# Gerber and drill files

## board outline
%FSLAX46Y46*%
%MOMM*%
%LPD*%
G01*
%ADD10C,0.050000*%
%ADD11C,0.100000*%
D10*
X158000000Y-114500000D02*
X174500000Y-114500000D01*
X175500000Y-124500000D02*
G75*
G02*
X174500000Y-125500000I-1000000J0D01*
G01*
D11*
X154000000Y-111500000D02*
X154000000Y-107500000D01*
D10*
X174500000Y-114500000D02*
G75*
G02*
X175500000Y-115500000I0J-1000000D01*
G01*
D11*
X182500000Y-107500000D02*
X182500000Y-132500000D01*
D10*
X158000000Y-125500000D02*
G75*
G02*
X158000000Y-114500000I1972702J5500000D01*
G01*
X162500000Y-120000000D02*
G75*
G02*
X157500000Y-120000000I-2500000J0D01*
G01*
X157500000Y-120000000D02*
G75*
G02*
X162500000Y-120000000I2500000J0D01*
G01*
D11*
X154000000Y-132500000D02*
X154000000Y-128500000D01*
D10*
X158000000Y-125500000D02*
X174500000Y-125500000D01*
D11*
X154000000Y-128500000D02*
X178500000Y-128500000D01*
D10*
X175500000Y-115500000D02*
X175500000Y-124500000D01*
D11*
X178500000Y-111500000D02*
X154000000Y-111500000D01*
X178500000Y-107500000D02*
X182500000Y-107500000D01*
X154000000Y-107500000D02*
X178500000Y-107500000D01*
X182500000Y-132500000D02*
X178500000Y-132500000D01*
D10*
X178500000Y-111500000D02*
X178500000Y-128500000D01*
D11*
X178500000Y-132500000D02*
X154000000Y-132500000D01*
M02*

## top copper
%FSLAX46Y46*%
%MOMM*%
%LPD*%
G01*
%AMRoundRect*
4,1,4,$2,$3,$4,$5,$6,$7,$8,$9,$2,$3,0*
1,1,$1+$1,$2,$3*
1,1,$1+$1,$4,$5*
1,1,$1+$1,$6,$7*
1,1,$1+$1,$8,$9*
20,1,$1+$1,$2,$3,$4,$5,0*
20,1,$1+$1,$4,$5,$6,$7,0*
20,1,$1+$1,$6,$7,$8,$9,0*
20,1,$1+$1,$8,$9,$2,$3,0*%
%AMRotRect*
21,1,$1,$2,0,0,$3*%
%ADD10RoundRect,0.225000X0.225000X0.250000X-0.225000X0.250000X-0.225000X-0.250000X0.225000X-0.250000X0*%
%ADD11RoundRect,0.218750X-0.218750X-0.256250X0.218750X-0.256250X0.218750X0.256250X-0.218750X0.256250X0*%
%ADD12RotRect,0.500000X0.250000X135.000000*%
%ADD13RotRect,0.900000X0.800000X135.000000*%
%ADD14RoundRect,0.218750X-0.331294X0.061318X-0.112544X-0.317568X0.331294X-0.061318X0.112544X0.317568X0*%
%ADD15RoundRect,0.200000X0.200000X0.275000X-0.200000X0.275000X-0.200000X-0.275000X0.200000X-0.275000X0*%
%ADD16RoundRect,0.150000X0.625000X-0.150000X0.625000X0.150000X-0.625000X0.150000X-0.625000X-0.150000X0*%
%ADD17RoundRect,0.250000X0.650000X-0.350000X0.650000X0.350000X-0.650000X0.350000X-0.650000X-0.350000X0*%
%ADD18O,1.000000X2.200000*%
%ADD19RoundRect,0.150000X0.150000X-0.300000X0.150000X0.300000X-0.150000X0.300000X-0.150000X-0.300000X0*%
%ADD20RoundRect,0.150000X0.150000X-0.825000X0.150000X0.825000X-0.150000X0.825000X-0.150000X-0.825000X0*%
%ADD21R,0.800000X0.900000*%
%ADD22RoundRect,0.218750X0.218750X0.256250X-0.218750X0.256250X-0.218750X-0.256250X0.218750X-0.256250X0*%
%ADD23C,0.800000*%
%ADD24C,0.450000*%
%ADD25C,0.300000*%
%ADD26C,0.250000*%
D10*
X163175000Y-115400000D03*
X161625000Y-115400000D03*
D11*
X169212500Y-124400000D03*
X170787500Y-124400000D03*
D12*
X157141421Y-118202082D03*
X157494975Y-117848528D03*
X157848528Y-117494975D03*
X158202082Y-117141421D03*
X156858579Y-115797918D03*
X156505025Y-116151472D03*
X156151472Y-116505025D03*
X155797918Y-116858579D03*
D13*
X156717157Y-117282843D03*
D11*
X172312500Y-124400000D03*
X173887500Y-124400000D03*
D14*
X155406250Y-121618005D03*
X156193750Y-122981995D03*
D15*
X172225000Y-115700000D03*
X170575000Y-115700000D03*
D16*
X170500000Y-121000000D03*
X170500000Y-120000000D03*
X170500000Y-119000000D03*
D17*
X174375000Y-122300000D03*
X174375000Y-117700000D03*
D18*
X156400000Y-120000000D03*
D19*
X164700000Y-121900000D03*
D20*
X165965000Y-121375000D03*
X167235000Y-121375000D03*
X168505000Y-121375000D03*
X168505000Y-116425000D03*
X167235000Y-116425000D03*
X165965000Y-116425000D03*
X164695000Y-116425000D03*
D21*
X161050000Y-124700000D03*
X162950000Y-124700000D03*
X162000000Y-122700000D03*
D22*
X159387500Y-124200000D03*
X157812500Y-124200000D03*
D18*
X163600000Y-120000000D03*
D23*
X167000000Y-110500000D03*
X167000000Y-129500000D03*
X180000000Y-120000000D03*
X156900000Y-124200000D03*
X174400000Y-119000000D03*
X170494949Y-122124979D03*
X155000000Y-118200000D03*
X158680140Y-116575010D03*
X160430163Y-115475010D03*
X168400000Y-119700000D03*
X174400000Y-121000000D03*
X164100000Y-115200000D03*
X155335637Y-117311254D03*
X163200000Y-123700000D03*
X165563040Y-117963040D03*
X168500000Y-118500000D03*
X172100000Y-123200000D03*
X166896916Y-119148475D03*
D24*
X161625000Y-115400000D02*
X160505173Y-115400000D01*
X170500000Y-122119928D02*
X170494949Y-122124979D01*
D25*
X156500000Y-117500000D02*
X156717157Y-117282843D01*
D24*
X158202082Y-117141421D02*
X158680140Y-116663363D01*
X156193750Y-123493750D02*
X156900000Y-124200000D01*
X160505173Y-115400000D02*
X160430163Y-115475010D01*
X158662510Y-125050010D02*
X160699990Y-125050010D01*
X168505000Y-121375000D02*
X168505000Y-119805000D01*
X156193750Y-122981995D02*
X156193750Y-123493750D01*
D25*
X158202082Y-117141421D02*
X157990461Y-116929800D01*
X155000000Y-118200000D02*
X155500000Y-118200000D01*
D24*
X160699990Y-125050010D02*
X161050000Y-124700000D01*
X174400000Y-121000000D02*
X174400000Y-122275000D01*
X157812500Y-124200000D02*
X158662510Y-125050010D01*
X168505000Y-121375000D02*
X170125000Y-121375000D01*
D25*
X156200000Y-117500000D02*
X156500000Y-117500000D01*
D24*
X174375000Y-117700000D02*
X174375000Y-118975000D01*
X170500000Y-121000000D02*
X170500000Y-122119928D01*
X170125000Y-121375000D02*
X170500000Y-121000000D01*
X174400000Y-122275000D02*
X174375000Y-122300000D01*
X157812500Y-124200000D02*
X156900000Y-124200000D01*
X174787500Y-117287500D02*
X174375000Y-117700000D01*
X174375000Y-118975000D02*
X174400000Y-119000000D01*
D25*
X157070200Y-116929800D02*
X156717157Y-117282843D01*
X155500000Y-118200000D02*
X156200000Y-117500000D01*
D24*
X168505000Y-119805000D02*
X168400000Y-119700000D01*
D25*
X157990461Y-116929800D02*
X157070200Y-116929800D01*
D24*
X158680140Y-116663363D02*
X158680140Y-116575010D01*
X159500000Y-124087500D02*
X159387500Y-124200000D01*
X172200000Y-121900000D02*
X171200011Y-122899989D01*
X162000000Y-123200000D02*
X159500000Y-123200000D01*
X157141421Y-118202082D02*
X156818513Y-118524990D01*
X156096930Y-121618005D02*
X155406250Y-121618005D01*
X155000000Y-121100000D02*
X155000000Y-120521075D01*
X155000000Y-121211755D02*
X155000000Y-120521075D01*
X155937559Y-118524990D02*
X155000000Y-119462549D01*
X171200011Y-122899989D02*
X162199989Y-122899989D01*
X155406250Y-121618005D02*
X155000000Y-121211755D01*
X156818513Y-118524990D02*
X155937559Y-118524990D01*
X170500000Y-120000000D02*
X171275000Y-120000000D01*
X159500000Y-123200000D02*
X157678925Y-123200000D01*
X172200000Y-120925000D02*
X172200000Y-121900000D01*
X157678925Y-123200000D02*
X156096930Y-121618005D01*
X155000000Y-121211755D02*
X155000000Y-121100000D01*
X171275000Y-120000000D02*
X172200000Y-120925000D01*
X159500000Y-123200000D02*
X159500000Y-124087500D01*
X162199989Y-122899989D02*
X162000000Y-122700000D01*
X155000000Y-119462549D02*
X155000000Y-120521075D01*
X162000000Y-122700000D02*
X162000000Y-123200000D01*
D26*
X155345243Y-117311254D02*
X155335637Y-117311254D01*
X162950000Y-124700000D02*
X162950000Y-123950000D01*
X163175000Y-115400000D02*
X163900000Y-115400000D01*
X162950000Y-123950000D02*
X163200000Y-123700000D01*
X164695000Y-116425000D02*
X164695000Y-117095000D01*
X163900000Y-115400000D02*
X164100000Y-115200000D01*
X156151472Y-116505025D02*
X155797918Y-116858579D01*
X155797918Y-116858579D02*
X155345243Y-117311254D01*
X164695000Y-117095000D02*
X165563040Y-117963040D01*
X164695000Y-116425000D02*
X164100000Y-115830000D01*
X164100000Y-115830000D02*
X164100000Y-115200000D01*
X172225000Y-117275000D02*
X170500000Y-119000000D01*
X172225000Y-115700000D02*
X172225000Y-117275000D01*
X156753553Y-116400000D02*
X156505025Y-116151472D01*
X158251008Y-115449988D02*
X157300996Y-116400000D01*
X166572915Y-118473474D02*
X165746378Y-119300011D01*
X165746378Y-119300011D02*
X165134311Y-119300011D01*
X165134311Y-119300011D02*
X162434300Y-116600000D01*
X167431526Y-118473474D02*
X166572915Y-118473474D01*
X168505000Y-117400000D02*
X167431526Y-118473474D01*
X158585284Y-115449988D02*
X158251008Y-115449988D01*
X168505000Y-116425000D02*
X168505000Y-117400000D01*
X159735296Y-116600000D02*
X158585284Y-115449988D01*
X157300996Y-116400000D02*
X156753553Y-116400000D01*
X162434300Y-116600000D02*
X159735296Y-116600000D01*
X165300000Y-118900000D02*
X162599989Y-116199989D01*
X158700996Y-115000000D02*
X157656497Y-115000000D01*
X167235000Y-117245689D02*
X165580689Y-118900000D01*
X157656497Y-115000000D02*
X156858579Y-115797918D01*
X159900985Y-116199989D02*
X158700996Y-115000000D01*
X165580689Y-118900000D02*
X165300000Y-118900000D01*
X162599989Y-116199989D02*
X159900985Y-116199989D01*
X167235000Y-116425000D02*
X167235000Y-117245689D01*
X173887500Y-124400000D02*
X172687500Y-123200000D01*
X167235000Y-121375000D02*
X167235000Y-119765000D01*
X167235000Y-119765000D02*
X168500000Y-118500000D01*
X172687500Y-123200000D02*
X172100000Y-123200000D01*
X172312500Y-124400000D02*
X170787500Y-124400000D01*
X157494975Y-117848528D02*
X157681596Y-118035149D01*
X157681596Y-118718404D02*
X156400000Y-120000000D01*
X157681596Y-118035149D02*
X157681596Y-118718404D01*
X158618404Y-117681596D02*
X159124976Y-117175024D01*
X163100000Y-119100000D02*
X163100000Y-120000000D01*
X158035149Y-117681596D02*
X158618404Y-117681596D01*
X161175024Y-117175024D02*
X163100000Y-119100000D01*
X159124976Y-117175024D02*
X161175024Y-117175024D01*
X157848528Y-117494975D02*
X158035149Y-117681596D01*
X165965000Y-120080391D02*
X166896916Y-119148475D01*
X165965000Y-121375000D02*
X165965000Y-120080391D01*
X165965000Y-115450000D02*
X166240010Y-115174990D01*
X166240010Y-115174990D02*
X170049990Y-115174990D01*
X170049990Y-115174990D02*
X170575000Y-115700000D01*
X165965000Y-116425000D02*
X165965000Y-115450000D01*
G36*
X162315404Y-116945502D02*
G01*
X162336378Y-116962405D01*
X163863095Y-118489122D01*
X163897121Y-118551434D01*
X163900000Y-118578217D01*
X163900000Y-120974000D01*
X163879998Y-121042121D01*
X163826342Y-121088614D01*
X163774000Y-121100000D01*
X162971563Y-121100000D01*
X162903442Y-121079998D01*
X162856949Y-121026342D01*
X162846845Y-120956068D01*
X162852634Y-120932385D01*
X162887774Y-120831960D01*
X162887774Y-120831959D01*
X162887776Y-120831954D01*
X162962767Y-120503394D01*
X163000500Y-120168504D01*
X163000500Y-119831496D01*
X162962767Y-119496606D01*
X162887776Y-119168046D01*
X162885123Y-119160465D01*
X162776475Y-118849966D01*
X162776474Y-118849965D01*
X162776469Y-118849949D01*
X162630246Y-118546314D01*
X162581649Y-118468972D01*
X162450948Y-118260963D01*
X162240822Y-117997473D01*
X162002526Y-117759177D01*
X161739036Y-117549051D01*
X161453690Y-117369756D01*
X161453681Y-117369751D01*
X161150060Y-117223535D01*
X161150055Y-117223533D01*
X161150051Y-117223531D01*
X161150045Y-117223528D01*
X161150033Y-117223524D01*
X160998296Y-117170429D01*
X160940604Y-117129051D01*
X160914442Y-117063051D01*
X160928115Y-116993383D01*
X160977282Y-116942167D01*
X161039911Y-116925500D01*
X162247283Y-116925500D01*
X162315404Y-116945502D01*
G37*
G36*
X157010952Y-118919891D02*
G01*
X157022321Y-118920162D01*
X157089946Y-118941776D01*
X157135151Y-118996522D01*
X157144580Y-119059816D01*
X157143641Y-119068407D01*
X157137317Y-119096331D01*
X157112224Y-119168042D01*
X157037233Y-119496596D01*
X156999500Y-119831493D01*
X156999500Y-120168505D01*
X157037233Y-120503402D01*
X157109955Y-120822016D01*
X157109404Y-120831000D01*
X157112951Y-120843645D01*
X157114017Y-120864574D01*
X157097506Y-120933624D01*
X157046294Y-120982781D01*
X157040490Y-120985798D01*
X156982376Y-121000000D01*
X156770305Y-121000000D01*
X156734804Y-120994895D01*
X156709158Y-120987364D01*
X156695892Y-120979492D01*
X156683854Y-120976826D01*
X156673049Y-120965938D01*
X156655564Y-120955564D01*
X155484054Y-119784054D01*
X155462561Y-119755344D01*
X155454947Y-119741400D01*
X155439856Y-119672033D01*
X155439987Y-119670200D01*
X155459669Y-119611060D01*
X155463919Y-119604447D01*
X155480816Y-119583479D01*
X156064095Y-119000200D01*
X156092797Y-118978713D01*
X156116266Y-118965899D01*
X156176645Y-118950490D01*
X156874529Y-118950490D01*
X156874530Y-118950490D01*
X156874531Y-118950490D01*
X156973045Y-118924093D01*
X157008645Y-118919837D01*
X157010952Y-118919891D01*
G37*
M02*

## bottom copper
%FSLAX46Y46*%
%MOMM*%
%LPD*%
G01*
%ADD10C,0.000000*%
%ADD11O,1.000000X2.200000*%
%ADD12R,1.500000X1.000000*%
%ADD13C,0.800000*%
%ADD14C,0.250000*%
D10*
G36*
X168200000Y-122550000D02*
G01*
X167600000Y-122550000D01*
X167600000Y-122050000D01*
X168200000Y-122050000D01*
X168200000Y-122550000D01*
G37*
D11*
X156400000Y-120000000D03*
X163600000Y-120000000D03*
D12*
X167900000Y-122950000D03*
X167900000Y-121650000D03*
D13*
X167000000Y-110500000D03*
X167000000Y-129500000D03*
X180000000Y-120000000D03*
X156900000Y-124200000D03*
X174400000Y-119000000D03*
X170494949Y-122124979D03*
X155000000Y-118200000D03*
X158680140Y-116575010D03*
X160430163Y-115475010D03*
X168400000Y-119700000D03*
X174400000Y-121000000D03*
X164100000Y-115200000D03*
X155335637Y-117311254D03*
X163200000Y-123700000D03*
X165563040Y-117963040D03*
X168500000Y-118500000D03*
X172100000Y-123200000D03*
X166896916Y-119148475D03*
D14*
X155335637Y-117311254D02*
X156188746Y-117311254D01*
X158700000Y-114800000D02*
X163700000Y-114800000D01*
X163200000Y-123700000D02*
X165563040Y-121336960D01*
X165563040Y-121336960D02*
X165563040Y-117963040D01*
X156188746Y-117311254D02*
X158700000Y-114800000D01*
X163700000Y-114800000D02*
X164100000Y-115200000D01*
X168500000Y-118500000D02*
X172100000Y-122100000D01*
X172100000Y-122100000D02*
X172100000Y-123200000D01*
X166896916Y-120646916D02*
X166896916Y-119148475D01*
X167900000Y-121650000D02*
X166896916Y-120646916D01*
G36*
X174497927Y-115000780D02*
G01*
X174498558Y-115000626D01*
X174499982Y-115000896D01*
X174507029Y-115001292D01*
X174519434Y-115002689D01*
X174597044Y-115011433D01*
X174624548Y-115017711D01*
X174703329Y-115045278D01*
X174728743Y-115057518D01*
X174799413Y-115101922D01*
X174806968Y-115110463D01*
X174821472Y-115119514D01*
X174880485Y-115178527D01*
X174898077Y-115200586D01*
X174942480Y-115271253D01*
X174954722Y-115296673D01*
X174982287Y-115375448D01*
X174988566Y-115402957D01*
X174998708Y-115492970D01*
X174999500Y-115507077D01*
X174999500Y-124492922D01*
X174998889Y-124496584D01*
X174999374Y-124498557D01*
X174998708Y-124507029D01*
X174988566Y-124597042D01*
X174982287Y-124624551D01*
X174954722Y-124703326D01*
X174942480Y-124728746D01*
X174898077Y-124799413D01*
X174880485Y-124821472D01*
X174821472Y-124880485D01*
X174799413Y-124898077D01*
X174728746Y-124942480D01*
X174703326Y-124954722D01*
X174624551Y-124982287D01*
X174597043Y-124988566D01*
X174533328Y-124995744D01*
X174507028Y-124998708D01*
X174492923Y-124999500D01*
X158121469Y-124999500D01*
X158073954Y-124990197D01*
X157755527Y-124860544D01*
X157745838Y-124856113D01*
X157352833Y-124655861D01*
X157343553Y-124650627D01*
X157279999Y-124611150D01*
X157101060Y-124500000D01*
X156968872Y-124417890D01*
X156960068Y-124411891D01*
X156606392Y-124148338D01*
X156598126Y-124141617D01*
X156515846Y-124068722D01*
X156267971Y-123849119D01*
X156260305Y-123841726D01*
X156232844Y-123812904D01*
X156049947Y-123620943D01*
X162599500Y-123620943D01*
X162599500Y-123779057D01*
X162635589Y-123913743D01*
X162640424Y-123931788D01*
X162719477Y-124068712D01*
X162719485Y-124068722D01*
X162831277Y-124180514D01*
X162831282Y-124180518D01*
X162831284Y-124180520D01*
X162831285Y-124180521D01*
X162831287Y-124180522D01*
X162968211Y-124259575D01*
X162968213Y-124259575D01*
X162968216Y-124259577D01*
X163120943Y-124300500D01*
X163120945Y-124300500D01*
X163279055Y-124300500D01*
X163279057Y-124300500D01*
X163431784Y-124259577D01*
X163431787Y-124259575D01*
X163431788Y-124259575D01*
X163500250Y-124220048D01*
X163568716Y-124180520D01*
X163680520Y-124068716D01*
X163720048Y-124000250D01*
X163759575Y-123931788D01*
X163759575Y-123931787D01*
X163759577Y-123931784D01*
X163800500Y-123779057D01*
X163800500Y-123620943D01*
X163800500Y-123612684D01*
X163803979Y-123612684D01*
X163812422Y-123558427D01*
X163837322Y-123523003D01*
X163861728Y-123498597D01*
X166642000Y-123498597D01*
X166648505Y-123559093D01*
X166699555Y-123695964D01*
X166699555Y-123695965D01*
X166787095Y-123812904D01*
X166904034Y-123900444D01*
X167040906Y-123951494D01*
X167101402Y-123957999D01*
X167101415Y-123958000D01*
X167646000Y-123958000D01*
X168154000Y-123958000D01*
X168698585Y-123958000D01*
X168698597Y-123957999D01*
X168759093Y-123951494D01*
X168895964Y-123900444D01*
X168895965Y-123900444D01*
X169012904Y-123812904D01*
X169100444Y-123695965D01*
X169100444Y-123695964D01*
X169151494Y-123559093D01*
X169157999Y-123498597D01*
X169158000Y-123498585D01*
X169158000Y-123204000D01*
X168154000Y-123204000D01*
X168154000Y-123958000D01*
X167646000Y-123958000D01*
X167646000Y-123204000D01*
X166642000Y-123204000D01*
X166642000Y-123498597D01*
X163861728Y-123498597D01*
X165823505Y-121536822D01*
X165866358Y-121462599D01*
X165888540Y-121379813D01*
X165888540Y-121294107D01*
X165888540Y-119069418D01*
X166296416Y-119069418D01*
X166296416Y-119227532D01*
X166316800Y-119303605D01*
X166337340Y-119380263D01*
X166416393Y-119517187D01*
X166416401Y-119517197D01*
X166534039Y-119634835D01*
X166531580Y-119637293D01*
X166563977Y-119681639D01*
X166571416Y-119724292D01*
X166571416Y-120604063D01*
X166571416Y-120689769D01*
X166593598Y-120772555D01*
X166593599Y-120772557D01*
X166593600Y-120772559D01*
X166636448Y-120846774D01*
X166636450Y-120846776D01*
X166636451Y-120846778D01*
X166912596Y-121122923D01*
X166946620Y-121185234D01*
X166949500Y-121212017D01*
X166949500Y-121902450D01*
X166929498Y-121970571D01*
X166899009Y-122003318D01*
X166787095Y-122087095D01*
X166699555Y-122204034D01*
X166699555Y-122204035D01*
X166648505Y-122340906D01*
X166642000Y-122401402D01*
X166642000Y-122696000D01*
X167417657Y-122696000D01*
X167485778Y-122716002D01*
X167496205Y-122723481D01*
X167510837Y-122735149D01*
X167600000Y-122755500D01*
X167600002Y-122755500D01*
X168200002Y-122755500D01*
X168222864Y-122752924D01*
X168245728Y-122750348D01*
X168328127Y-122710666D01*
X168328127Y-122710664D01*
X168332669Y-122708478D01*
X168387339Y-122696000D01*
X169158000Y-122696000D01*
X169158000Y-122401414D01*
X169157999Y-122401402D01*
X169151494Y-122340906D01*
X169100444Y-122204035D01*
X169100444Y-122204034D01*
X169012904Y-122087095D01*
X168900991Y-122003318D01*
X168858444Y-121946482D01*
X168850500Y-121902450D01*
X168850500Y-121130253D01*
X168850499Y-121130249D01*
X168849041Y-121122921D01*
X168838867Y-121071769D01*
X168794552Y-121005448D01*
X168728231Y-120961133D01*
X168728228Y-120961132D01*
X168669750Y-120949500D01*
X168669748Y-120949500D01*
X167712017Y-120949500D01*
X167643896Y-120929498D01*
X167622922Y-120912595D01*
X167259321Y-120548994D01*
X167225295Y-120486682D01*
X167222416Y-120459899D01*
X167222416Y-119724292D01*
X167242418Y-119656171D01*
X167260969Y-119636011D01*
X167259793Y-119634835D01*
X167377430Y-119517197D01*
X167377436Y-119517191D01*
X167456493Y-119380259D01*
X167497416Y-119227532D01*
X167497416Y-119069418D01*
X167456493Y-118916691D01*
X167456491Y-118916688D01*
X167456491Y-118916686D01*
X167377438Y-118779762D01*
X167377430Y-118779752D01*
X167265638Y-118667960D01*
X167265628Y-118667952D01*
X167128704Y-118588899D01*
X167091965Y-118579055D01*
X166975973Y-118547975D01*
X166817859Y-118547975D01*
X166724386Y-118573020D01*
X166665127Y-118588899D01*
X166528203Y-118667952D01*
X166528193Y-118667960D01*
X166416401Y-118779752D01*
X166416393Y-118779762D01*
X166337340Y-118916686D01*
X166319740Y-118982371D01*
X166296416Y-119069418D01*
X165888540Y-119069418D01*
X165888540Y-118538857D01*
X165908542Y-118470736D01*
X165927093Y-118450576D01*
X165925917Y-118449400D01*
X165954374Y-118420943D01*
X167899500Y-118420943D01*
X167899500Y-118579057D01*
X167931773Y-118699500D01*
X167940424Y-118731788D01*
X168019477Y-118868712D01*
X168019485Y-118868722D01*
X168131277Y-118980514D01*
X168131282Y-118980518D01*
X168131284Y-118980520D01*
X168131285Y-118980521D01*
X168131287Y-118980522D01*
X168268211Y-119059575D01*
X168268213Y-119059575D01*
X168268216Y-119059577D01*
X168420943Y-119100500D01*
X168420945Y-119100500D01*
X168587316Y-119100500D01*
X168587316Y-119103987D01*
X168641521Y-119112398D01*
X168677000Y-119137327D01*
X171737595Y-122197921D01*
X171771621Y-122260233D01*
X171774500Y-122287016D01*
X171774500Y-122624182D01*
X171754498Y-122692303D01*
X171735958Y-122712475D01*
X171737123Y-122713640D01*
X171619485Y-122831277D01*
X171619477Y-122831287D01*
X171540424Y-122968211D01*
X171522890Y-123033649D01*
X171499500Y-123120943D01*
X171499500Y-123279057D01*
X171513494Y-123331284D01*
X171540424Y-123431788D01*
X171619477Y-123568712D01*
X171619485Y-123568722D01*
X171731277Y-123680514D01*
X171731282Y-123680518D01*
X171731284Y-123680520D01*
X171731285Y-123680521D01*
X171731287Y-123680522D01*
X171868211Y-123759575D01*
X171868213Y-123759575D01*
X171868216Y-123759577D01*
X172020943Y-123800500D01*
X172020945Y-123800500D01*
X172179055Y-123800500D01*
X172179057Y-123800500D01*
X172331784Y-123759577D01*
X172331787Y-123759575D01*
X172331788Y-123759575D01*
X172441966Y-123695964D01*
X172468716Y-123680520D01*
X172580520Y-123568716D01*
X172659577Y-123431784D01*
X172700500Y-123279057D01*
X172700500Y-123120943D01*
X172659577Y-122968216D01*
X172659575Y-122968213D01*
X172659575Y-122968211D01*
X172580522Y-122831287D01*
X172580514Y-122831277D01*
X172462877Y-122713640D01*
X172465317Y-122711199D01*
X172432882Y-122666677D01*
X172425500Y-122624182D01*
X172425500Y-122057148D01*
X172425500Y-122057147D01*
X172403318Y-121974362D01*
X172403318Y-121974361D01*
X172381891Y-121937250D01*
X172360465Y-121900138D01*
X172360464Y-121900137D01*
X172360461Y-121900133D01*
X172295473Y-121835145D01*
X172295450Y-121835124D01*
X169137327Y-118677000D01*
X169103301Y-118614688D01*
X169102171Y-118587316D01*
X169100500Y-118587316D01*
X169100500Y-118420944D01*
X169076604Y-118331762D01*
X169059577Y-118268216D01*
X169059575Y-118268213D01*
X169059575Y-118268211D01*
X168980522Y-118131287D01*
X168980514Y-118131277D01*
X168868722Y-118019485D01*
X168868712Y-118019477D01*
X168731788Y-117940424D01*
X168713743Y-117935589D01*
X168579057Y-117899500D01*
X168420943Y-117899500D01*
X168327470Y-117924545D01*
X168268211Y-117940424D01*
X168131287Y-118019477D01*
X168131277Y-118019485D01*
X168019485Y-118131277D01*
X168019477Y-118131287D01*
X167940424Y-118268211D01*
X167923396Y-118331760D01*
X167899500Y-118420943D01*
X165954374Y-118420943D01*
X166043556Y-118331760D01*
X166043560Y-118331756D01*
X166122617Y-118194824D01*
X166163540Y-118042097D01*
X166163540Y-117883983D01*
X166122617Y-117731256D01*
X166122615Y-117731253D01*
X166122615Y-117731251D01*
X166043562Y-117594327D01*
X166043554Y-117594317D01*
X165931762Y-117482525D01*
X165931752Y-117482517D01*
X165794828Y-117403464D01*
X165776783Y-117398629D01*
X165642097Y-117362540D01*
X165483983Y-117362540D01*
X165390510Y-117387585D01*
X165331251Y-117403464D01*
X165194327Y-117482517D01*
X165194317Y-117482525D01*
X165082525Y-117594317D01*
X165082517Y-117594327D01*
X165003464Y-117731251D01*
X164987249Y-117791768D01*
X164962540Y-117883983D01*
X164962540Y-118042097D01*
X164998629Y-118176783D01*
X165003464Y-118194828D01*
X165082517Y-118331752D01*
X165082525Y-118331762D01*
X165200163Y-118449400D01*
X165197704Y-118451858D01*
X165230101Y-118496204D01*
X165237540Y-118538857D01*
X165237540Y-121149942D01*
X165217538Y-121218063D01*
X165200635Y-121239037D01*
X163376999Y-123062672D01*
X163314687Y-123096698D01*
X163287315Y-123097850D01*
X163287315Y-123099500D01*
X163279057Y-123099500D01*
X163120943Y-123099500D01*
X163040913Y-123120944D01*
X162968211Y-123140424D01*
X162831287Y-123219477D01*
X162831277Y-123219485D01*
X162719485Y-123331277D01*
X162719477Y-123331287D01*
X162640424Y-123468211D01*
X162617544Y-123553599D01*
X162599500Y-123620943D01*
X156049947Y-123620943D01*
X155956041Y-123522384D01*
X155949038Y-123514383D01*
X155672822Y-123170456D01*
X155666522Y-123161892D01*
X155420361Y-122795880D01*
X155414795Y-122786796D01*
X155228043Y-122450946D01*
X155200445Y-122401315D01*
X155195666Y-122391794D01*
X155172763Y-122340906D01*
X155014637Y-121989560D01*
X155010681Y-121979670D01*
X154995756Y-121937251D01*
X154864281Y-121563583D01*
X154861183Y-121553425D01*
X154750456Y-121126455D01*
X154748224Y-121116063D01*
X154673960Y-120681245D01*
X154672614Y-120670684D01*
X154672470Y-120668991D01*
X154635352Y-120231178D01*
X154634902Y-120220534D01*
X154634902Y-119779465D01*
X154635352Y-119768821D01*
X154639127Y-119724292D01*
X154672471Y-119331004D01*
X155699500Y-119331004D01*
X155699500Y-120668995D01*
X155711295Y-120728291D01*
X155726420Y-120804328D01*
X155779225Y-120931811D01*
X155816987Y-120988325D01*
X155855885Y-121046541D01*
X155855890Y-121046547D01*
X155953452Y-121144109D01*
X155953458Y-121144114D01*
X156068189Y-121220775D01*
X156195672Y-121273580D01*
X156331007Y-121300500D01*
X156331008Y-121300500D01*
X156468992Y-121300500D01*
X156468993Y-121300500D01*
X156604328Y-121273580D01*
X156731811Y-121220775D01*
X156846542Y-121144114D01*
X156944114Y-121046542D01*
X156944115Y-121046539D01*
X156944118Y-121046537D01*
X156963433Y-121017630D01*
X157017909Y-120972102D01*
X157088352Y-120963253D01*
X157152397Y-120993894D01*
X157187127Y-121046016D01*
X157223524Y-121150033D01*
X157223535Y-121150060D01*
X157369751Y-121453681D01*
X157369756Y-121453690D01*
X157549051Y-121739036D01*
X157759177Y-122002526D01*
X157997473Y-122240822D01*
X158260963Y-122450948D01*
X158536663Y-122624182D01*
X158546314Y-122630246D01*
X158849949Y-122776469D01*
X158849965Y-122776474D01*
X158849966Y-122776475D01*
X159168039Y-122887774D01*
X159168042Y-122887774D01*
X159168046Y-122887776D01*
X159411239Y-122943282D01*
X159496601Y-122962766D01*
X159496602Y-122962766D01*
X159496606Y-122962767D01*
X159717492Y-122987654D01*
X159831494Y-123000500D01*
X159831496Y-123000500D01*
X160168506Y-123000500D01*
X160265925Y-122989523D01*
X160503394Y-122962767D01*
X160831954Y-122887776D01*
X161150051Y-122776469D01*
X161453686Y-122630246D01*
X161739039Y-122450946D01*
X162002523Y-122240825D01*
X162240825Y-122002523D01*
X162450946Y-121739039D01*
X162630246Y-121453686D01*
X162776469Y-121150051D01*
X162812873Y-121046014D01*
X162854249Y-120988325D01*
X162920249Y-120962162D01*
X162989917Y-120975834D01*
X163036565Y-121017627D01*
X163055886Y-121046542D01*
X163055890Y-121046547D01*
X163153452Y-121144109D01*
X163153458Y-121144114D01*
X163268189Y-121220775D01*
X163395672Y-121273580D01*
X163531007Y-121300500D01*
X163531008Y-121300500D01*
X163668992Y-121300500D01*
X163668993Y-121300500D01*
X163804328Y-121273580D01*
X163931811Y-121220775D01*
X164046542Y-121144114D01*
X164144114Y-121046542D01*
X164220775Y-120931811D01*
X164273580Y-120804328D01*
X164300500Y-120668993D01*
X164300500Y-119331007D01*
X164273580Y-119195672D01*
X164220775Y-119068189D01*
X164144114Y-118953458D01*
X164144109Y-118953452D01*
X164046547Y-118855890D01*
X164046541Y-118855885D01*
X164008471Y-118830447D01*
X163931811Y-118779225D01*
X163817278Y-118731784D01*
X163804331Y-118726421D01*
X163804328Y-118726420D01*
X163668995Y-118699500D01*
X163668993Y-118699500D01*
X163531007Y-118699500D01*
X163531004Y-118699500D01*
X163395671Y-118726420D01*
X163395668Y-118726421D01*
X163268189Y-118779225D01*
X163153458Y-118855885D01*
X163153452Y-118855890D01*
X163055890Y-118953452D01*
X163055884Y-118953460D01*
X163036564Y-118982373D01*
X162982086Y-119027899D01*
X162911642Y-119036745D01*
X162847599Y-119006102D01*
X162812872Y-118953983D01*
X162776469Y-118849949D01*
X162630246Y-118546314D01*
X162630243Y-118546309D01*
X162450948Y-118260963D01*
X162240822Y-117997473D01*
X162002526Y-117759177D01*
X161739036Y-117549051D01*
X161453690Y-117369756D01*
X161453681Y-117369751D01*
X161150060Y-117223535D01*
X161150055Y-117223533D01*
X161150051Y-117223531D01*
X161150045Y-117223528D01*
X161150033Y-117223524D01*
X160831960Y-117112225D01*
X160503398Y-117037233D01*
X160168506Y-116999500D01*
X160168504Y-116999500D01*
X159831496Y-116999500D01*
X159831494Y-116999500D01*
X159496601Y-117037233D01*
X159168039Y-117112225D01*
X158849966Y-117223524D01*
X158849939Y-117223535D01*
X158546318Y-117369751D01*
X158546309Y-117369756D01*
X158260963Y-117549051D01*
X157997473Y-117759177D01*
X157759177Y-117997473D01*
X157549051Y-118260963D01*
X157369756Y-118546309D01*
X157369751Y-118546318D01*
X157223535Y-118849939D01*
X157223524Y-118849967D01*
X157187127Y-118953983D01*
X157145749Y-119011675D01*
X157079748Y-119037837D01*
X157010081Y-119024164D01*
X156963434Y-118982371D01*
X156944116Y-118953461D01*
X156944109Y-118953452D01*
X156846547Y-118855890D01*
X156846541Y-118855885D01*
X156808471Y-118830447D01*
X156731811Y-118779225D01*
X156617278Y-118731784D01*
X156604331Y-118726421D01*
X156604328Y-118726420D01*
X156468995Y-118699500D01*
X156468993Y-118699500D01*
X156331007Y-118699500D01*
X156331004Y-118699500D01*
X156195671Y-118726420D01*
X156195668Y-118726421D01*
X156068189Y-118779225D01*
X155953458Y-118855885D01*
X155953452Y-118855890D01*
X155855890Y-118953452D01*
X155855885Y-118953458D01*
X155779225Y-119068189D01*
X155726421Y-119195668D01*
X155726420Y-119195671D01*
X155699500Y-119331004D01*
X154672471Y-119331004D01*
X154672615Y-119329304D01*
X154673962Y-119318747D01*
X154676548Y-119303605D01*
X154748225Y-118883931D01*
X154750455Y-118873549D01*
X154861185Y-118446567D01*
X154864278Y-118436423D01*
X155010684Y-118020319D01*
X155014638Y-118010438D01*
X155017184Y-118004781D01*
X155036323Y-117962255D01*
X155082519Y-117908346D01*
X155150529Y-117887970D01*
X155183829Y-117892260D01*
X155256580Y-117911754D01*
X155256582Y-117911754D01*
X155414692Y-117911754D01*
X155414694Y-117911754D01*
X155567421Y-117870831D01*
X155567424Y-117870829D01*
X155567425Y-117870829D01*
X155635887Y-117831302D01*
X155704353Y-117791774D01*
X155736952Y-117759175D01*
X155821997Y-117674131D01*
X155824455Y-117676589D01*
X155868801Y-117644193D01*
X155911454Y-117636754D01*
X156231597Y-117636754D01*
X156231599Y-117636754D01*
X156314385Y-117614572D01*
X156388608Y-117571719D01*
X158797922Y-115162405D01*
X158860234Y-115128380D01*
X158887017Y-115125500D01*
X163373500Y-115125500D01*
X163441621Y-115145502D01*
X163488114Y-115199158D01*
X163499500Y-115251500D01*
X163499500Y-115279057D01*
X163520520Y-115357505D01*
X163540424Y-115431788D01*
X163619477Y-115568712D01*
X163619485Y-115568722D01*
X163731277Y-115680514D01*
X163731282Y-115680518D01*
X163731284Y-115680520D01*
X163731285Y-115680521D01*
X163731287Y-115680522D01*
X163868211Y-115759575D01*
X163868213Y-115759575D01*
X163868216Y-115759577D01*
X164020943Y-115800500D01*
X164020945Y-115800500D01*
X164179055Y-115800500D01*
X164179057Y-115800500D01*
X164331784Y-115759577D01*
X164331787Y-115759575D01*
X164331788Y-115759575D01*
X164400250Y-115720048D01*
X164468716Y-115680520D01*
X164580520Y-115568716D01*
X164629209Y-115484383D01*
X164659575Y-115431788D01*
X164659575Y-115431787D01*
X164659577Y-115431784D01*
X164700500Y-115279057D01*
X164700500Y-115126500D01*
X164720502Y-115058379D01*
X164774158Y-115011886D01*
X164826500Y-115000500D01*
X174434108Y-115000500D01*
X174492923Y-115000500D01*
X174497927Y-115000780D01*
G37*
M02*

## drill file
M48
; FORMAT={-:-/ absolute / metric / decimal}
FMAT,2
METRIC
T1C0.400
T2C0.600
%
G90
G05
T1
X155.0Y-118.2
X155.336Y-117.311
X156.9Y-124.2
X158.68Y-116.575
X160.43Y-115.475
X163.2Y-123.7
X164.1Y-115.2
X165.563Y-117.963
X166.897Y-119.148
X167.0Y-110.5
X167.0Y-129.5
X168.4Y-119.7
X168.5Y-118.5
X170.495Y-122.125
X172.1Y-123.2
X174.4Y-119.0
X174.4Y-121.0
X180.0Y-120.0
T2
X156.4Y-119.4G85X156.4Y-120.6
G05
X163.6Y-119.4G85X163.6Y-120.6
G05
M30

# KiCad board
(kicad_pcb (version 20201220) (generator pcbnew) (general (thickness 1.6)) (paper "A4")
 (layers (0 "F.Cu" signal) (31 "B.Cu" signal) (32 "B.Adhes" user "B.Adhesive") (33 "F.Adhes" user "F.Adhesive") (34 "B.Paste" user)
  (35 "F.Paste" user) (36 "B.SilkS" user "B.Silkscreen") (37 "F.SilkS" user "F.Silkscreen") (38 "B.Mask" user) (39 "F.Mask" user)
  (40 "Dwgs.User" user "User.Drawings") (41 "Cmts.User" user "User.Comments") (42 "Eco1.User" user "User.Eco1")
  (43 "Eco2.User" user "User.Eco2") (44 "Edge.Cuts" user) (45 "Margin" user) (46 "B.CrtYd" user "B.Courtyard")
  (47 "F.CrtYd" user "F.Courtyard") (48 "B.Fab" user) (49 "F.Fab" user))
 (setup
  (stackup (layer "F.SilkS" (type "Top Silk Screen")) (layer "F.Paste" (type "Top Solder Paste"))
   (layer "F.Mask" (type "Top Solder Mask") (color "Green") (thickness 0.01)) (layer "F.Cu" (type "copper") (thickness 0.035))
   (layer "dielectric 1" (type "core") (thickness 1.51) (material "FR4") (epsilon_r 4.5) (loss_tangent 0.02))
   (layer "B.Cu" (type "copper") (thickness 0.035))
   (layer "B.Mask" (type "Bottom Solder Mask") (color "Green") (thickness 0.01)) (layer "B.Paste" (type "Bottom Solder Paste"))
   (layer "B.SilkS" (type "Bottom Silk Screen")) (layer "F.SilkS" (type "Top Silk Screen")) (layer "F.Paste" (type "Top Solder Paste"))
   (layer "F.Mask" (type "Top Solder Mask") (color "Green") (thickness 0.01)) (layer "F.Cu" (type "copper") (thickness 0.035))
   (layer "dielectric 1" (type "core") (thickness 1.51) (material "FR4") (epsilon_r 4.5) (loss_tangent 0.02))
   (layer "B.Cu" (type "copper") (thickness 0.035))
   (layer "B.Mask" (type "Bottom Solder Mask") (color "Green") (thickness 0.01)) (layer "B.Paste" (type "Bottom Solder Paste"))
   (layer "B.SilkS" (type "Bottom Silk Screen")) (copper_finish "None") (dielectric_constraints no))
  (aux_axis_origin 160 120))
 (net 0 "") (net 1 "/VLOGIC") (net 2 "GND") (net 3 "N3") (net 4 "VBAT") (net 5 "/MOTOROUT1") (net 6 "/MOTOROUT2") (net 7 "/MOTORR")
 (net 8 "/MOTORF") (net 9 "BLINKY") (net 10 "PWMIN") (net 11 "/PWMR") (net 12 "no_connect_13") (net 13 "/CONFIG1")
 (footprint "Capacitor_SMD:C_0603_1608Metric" (layer "F.Cu") (at 162.4 115.4 180)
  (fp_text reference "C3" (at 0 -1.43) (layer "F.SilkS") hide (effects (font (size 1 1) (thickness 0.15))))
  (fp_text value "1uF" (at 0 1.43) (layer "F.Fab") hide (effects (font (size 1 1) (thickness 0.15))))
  (pad "1" smd roundrect (at -0.775 0 180) (size 0.9 0.95) (layers "F.Cu" "F.Paste" "F.Mask") (roundrect_rratio 0.25) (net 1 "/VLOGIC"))
  (pad "2" smd roundrect (at 0.775 0 180) (size 0.9 0.95) (layers "F.Cu" "F.Paste" "F.Mask") (roundrect_rratio 0.25) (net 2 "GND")))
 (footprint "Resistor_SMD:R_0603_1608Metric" (layer "F.Cu") (at 170 124.4)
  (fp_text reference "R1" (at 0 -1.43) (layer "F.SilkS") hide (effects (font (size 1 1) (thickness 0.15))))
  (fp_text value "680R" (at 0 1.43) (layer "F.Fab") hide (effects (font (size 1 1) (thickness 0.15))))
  (pad "1" smd roundrect (at -0.7875 0) (size 0.875 0.95) (layers "F.Cu" "F.Paste" "F.Mask") (roundrect_rratio 0.25) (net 2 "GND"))
  (pad "2" smd roundrect (at 0.7875 0) (size 0.875 0.95) (layers "F.Cu" "F.Paste" "F.Mask") (roundrect_rratio 0.25) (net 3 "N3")))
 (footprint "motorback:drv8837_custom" (layer "F.Cu") (at 157 117 135)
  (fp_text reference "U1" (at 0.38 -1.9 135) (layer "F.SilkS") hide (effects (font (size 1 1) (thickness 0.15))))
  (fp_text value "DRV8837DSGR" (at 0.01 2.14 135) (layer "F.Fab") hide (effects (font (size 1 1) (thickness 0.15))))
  (pad "" smd rect (at 0 -0.4 135) (size 0.75 0.65) (layers "F.Paste"))
  (pad "1" smd rect (at -0.95 -0.75 135) (size 0.5 0.25) (layers "F.Cu" "F.Paste" "F.Mask") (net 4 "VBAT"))
  (pad "2" smd rect (at -0.95 -0.25 135) (size 0.5 0.25) (layers "F.Cu" "F.Paste" "F.Mask") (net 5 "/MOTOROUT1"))
  (pad "3" smd rect (at -0.95 0.25 135) (size 0.5 0.25) (layers "F.Cu" "F.Paste" "F.Mask") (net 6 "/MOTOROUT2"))
  (pad "4" smd rect (at -0.95 0.75 135) (size 0.5 0.25) (layers "F.Cu" "F.Paste" "F.Mask") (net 2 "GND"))
  (pad "5" smd rect (at 0.95 0.75 135) (size 0.5 0.25) (layers "F.Cu" "F.Paste" "F.Mask") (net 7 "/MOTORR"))
  (pad "6" smd rect (at 0.95 0.25 135) (size 0.5 0.25) (layers "F.Cu" "F.Paste" "F.Mask") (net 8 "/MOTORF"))
  (pad "7" smd rect (at 0.95 -0.25 135) (size 0.5 0.25) (layers "F.Cu" "F.Paste" "F.Mask") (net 1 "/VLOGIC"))
  (pad "8" smd rect (at 0.95 -0.75 135) (size 0.5 0.25) (layers "F.Cu" "F.Paste" "F.Mask") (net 1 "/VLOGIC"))
  (pad "9" smd rect (at 0 -0.4 135) (size 0.9 0.8) (layers "F.Cu" "F.Mask") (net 2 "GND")))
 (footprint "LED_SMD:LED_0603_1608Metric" (layer "F.Cu") (at 173.1 124.4)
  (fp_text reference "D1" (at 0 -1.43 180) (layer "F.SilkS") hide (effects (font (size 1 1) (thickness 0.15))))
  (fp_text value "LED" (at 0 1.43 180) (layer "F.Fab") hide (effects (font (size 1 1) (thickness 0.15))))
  (pad "1" smd roundrect (at -0.7875 0) (size 0.875 0.95) (layers "F.Cu" "F.Paste" "F.Mask") (roundrect_rratio 0.25) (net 3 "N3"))
  (pad "2" smd roundrect (at 0.7875 0) (size 0.875 0.95) (layers "F.Cu" "F.Paste" "F.Mask") (roundrect_rratio 0.25) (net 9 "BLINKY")))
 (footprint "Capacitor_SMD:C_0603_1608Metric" (layer "F.Cu") (at 155.8 122.3 -60)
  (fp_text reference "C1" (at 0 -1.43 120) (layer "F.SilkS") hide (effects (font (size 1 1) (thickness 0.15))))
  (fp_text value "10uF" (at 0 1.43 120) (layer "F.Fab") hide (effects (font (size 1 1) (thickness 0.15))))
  (pad "1" smd roundrect (at -0.7875 0 300) (size 0.875 0.95) (layers "F.Cu" "F.Paste" "F.Mask") (roundrect_rratio 0.25) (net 4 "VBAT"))
  (pad "2" smd roundrect (at 0.7875 0 300) (size 0.875 0.95) (layers "F.Cu" "F.Paste" "F.Mask") (roundrect_rratio 0.25) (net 2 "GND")))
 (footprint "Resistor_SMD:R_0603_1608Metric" (layer "F.Cu") (at 171.4 115.7 180)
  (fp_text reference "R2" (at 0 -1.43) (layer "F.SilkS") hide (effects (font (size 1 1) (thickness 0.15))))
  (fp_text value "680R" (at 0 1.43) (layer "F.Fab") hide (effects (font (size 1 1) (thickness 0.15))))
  (pad "1" smd roundrect (at -0.825 0 180) (size 0.8 0.95) (layers "F.Cu" "F.Paste" "F.Mask") (roundrect_rratio 0.25) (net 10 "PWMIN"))
  (pad "2" smd roundrect (at 0.825 0 180) (size 0.8 0.95) (layers "F.Cu" "F.Paste" "F.Mask") (roundrect_rratio 0.25) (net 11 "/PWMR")))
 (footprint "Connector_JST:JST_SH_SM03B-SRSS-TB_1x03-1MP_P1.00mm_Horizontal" (layer "F.Cu") (at 172.5 120 90)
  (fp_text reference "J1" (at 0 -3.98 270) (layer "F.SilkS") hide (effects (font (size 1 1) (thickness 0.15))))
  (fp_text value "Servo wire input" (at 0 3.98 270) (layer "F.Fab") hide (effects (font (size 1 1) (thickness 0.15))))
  (pad "1" smd roundrect (at -1 -2 90) (size 0.6 1.55) (layers "F.Cu" "F.Paste" "F.Mask") (roundrect_rratio 0.25) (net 2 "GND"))
  (pad "2" smd roundrect (at 0 -2 90) (size 0.6 1.55) (layers "F.Cu" "F.Paste" "F.Mask") (roundrect_rratio 0.25) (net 4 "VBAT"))
  (pad "3" smd roundrect (at 1 -2 90) (size 0.6 1.55) (layers "F.Cu" "F.Paste" "F.Mask") (roundrect_rratio 0.25) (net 10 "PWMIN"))
  (pad "MP" smd roundrect (at -2.3 1.875 90) (size 1.2 1.8) (layers "F.Cu" "F.Paste" "F.Mask") (roundrect_rratio 0.2083333333333333)
   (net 2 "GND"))
  (pad "MP" smd roundrect (at 2.3 1.875 90) (size 1.2 1.8) (layers "F.Cu" "F.Paste" "F.Mask") (roundrect_rratio 0.2083333333333333)
   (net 2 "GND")))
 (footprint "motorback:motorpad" (layer "F.Cu") (at 156.4 120)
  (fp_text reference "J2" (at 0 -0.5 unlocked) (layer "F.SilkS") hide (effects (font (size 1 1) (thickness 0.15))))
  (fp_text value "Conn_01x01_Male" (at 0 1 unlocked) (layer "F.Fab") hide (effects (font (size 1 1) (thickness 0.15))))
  (pad "1" thru_hole oval (at 0 0) (size 1 2.2) (drill oval 0.6 1.8) (layers *.Cu *.Mask) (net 5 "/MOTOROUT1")))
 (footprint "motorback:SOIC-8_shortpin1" (layer "F.Cu") (at 166.6 118.9 90)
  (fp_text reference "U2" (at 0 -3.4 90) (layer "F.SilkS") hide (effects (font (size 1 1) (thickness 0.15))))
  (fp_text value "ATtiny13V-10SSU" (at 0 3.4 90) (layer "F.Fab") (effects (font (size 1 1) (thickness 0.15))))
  (pad "1" smd roundrect (at -3 -1.9 90) (size 0.9 0.6) (layers "F.Cu" "F.Paste" "F.Mask") (roundrect_rratio 0.25) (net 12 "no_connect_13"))
  (pad "2" smd roundrect (at -2.475 -0.635 90) (size 1.95 0.6) (layers "F.Cu" "F.Paste" "F.Mask") (roundrect_rratio 0.25)
   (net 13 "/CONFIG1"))
  (pad "3" smd roundrect (at -2.475 0.635 90) (size 1.95 0.6) (layers "F.Cu" "F.Paste" "F.Mask") (roundrect_rratio 0.25) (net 9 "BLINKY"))
  (pad "4" smd roundrect (at -2.475 1.905 90) (size 1.95 0.6) (layers "F.Cu" "F.Paste" "F.Mask") (roundrect_rratio 0.25) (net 2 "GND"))
  (pad "5" smd roundrect (at 2.475 1.905 90) (size 1.95 0.6) (layers "F.Cu" "F.Paste" "F.Mask") (roundrect_rratio 0.25) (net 8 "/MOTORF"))
  (pad "6" smd roundrect (at 2.475 0.635 90) (size 1.95 0.6) (layers "F.Cu" "F.Paste" "F.Mask") (roundrect_rratio 0.25) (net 7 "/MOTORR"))
  (pad "7" smd roundrect (at 2.475 -0.635 90) (size 1.95 0.6) (layers "F.Cu" "F.Paste" "F.Mask") (roundrect_rratio 0.25) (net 11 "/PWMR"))
  (pad "8" smd roundrect (at 2.475 -1.905 90) (size 1.95 0.6) (layers "F.Cu" "F.Paste" "F.Mask") (roundrect_rratio 0.25) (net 1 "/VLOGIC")))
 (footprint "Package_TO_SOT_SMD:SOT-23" (layer "F.Cu") (at 162 123.7 90)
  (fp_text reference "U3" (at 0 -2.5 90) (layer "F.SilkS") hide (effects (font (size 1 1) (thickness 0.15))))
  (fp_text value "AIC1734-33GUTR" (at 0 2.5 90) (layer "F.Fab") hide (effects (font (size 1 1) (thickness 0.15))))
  (pad "1" smd rect (at -1 -0.95 90) (size 0.9 0.8) (layers "F.Cu" "F.Paste" "F.Mask") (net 2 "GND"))
  (pad "2" smd rect (at -1 0.95 90) (size 0.9 0.8) (layers "F.Cu" "F.Paste" "F.Mask") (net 1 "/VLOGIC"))
  (pad "3" smd rect (at 1 0 90) (size 0.9 0.8) (layers "F.Cu" "F.Paste" "F.Mask") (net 4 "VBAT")))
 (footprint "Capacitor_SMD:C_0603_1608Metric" (layer "F.Cu") (at 158.6 124.2 180)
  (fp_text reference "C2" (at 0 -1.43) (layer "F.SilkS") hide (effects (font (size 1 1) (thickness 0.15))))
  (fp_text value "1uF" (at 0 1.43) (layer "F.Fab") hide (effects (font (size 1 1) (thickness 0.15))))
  (pad "1" smd roundrect (at -0.7875 0 180) (size 0.875 0.95) (layers "F.Cu" "F.Paste" "F.Mask") (roundrect_rratio 0.25) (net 4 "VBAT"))
  (pad "2" smd roundrect (at 0.7875 0 180) (size 0.875 0.95) (layers "F.Cu" "F.Paste" "F.Mask") (roundrect_rratio 0.25) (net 2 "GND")))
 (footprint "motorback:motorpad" (layer "F.Cu") (at 163.6 120)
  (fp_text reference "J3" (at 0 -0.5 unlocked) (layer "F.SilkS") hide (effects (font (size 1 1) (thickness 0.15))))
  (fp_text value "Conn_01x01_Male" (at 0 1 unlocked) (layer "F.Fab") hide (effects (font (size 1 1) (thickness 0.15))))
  (pad "1" thru_hole oval (at 0 0) (size 1 2.2) (drill oval 0.6 1.8) (layers *.Cu *.Mask) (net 6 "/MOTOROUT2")))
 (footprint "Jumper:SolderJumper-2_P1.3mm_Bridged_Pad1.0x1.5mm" (layer "B.Cu") (at 167.9 122.3 90)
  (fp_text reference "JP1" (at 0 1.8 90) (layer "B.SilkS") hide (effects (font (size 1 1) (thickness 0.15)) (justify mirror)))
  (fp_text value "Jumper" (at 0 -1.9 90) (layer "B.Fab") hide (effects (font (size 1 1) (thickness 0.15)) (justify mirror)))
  (fp_poly (pts (xy -0.25 0.3) (xy 0.25 0.3) (xy 0.25 -0.3) (xy -0.25 -0.3)) (layer "B.Cu") (width 0) (fill solid))
  (pad "1" smd rect (at -0.65 0 90) (size 1 1.5) (layers "B.Cu" "B.Mask") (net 2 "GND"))
  (pad "2" smd rect (at 0.65 0 90) (size 1 1.5) (layers "B.Cu" "B.Mask") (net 13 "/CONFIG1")))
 (gr_line (start 158 114.5) (end 174.5 114.5) (layer "Edge.Cuts") (width 0.05))
 (gr_arc (start 174.5 124.5) (end 174.5 125.5) (angle -90) (layer "Edge.Cuts") (width 0.05))
 (gr_line (start 154 111.5) (end 154 107.5) (layer "Edge.Cuts") (width 0.1))
 (gr_arc (start 174.5 115.5) (end 175.5 115.5) (angle -90) (layer "Edge.Cuts") (width 0.05))
 (gr_line (start 182.5 107.5) (end 182.5 132.5) (layer "Edge.Cuts") (width 0.1))
 (gr_arc (start 159.972702 120) (end 158 114.5) (angle -140.5369116) (layer "Edge.Cuts") (width 0.05))
 (gr_circle (center 160 120) (end 162.5 120) (layer "Edge.Cuts") (width 0.05) (fill none))
 (gr_line (start 154 132.5) (end 154 128.5) (layer "Edge.Cuts") (width 0.1))
 (gr_line (start 158 125.5) (end 174.5 125.5) (layer "Edge.Cuts") (width 0.05))
 (gr_line (start 154 128.5) (end 178.5 128.5) (layer "Edge.Cuts") (width 0.1))
 (gr_line (start 175.5 115.5) (end 175.5 124.5) (layer "Edge.Cuts") (width 0.05))
 (gr_line (start 178.5 111.5) (end 154 111.5) (layer "Edge.Cuts") (width 0.1))
 (gr_line (start 178.5 107.5) (end 182.5 107.5) (layer "Edge.Cuts") (width 0.1))
 (gr_line (start 154 107.5) (end 178.5 107.5) (layer "Edge.Cuts") (width 0.1))
 (gr_line (start 182.5 132.5) (end 178.5 132.5) (layer "Edge.Cuts") (width 0.1))
 (gr_line (start 178.5 111.5) (end 178.5 128.5) (layer "Edge.Cuts") (width 0.05))
 (gr_line (start 178.5 132.5) (end 154 132.5) (layer "Edge.Cuts") (width 0.1))
 (via (at 167 110.5) (size 0.8) (drill 0.4) (layers "F.Cu" "B.Cu") (free) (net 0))
 (via (at 167 129.5) (size 0.8) (drill 0.4) (layers "F.Cu" "B.Cu") (free) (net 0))
 (via (at 180 120) (size 0.8) (drill 0.4) (layers "F.Cu" "B.Cu") (free) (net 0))
 (segment (start 161.625 115.4) (end 160.505173 115.4) (width 0.45) (layer "F.Cu") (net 2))
 (segment (start 170.5 122.119928) (end 170.494949 122.124979) (width 0.45) (layer "F.Cu") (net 2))
 (segment (start 156.5 117.5) (end 156.717157 117.282843) (width 0.3) (layer "F.Cu") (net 2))
 (segment (start 158.202082 117.141421) (end 158.68014 116.663363) (width 0.45) (layer "F.Cu") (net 2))
 (segment (start 156.19375 123.49375) (end 156.9 124.2) (width 0.45) (layer "F.Cu") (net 2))
 (segment (start 160.505173 115.4) (end 160.430163 115.47501) (width 0.45) (layer "F.Cu") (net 2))
 (segment (start 158.66251 125.05001) (end 160.69999 125.05001) (width 0.45) (layer "F.Cu") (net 2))
 (segment (start 168.505 121.375) (end 168.505 119.805) (width 0.45) (layer "F.Cu") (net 2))
 (segment (start 156.19375 122.981995) (end 156.19375 123.49375) (width 0.45) (layer "F.Cu") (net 2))
 (segment (start 158.202082 117.141421) (end 157.990461 116.9298) (width 0.3) (layer "F.Cu") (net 2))
 (segment (start 155 118.2) (end 155.5 118.2) (width 0.3) (layer "F.Cu") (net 2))
 (segment (start 160.69999 125.05001) (end 161.05 124.7) (width 0.45) (layer "F.Cu") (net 2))
 (segment (start 174.4 121) (end 174.4 122.275) (width 0.45) (layer "F.Cu") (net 2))
 (segment (start 157.8125 124.2) (end 158.66251 125.05001) (width 0.45) (layer "F.Cu") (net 2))
 (segment (start 168.505 121.375) (end 170.125 121.375) (width 0.45) (layer "F.Cu") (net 2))
 (segment (start 156.2 117.5) (end 156.5 117.5) (width 0.3) (layer "F.Cu") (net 2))
 (segment (start 174.375 117.7) (end 174.375 118.975) (width 0.45) (layer "F.Cu") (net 2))
 (segment (start 170.5 121) (end 170.5 122.119928) (width 0.45) (layer "F.Cu") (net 2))
 (segment (start 170.125 121.375) (end 170.5 121) (width 0.45) (layer "F.Cu") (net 2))
 (segment (start 174.4 122.275) (end 174.375 122.3) (width 0.45) (layer "F.Cu") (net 2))
 (segment (start 157.8125 124.2) (end 156.9 124.2) (width 0.45) (layer "F.Cu") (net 2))
 (segment (start 174.7875 117.2875) (end 174.375 117.7) (width 0.45) (layer "F.Cu") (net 2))
 (segment (start 174.375 118.975) (end 174.4 119) (width 0.45) (layer "F.Cu") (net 2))
 (segment (start 157.0702 116.9298) (end 156.717157 117.282843) (width 0.3) (layer "F.Cu") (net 2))
 (segment (start 155.5 118.2) (end 156.2 117.5) (width 0.3) (layer "F.Cu") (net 2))
 (segment (start 168.505 119.805) (end 168.4 119.7) (width 0.45) (layer "F.Cu") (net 2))
 (segment (start 157.990461 116.9298) (end 157.0702 116.9298) (width 0.3) (layer "F.Cu") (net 2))
 (segment (start 158.68014 116.663363) (end 158.68014 116.57501) (width 0.45) (layer "F.Cu") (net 2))
 (via (at 156.9 124.2) (size 0.8) (drill 0.4) (layers "F.Cu" "B.Cu") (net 2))
 (via (at 174.4 119) (size 0.8) (drill 0.4) (layers "F.Cu" "B.Cu") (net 2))
 (via (at 170.494949 122.124979) (size 0.8) (drill 0.4) (layers "F.Cu" "B.Cu") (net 2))
 (via (at 155 118.2) (size 0.8) (drill 0.4) (layers "F.Cu" "B.Cu") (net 2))
 (via (at 158.68014 116.57501) (size 0.8) (drill 0.4) (layers "F.Cu" "B.Cu") (free) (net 2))
 (via (at 160.430163 115.47501) (size 0.8) (drill 0.4) (layers "F.Cu" "B.Cu") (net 2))
 (via (at 168.4 119.7) (size 0.8) (drill 0.4) (layers "F.Cu" "B.Cu") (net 2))
 (via (at 174.4 121) (size 0.8) (drill 0.4) (layers "F.Cu" "B.Cu") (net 2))
 (segment (start 159.5 124.0875) (end 159.3875 124.2) (width 0.45) (layer "F.Cu") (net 4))
 (segment (start 172.2 121.9) (end 171.200011 122.899989) (width 0.45) (layer "F.Cu") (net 4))
 (segment (start 162 123.2) (end 159.5 123.2) (width 0.45) (layer "F.Cu") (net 4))
 (segment (start 157.141421 118.202082) (end 156.818513 118.52499) (width 0.45) (layer "F.Cu") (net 4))
 (segment (start 156.09693 121.618005) (end 155.40625 121.618005) (width 0.45) (layer "F.Cu") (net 4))
 (segment (start 155 121.1) (end 155 120.521075) (width 0.45) (layer "F.Cu") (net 4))
 (segment (start 155 121.211755) (end 155 120.521075) (width 0.45) (layer "F.Cu") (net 4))
 (segment (start 155.937559 118.52499) (end 155 119.462549) (width 0.45) (layer "F.Cu") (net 4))
 (segment (start 171.200011 122.899989) (end 162.199989 122.899989) (width 0.45) (layer "F.Cu") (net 4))
 (segment (start 155.40625 121.618005) (end 155 121.211755) (width 0.45) (layer "F.Cu") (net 4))
 (segment (start 156.818513 118.52499) (end 155.937559 118.52499) (width 0.45) (layer "F.Cu") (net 4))
 (segment (start 170.5 120) (end 171.275 120) (width 0.45) (layer "F.Cu") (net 4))
 (segment (start 159.5 123.2) (end 157.678925 123.2) (width 0.45) (layer "F.Cu") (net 4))
 (segment (start 172.2 120.925) (end 172.2 121.9) (width 0.45) (layer "F.Cu") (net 4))
 (segment (start 157.678925 123.2) (end 156.09693 121.618005) (width 0.45) (layer "F.Cu") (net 4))
 (segment (start 155 121.211755) (end 155 121.1) (width 0.45) (layer "F.Cu") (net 4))
 (segment (start 171.275 120) (end 172.2 120.925) (width 0.45) (layer "F.Cu") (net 4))
 (segment (start 159.5 123.2) (end 159.5 124.0875) (width 0.45) (layer "F.Cu") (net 4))
 (segment (start 162.199989 122.899989) (end 162 122.7) (width 0.45) (layer "F.Cu") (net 4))
 (segment (start 155 119.462549) (end 155 120.521075) (width 0.45) (layer "F.Cu") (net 4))
 (segment (start 162 122.7) (end 162 123.2) (width 0.45) (layer "F.Cu") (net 4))
 (segment (start 155.345243 117.311254) (end 155.335637 117.311254) (width 0.25) (layer "F.Cu") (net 1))
 (segment (start 162.95 124.7) (end 162.95 123.95) (width 0.25) (layer "F.Cu") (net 1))
 (segment (start 163.175 115.4) (end 163.9 115.4) (width 0.25) (layer "F.Cu") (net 1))
 (segment (start 162.95 123.95) (end 163.2 123.7) (width 0.25) (layer "F.Cu") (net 1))
 (segment (start 164.695 116.425) (end 164.695 117.095) (width 0.25) (layer "F.Cu") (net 1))
 (segment (start 163.9 115.4) (end 164.1 115.2) (width 0.25) (layer "F.Cu") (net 1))
 (segment (start 156.151472 116.505025) (end 155.797918 116.858579) (width 0.25) (layer "F.Cu") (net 1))
 (segment (start 155.797918 116.858579) (end 155.345243 117.311254) (width 0.25) (layer "F.Cu") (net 1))
 (segment (start 164.695 117.095) (end 165.56304 117.96304) (width 0.25) (layer "F.Cu") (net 1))
 (segment (start 164.695 116.425) (end 164.1 115.83) (width 0.25) (layer "F.Cu") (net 1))
 (segment (start 164.1 115.83) (end 164.1 115.2) (width 0.25) (layer "F.Cu") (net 1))
 (via (at 164.1 115.2) (size 0.8) (drill 0.4) (layers "F.Cu" "B.Cu") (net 1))
 (via (at 155.335637 117.311254) (size 0.8) (drill 0.4) (layers "F.Cu" "B.Cu") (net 1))
 (via (at 163.2 123.7) (size 0.8) (drill 0.4) (layers "F.Cu" "B.Cu") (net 1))
 (via (at 165.56304 117.96304) (size 0.8) (drill 0.4) (layers "F.Cu" "B.Cu") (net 1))
 (segment (start 155.335637 117.311254) (end 156.188746 117.311254) (width 0.25) (layer "B.Cu") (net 1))
 (segment (start 158.7 114.8) (end 163.7 114.8) (width 0.25) (layer "B.Cu") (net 1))
 (segment (start 163.2 123.7) (end 165.56304 121.33696) (width 0.25) (layer "B.Cu") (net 1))
 (segment (start 165.56304 121.33696) (end 165.56304 117.96304) (width 0.25) (layer "B.Cu") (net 1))
 (segment (start 156.188746 117.311254) (end 158.7 114.8) (width 0.25) (layer "B.Cu") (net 1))
 (segment (start 163.7 114.8) (end 164.1 115.2) (width 0.25) (layer "B.Cu") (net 1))
 (segment (start 172.225 117.275) (end 170.5 119) (width 0.25) (layer "F.Cu") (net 10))
 (segment (start 172.225 115.7) (end 172.225 117.275) (width 0.25) (layer "F.Cu") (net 10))
 (segment (start 156.753553 116.4) (end 156.505025 116.151472) (width 0.25) (layer "F.Cu") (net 8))
 (segment (start 158.251008 115.449988) (end 157.300996 116.4) (width 0.25) (layer "F.Cu") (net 8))
 (segment (start 166.572915 118.473474) (end 165.746378 119.300011) (width 0.25) (layer "F.Cu") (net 8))
 (segment (start 165.746378 119.300011) (end 165.134311 119.300011) (width 0.25) (layer "F.Cu") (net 8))
 (segment (start 165.134311 119.300011) (end 162.4343 116.6) (width 0.25) (layer "F.Cu") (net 8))
 (segment (start 167.431526 118.473474) (end 166.572915 118.473474) (width 0.25) (layer "F.Cu") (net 8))
 (segment (start 168.505 117.4) (end 167.431526 118.473474) (width 0.25) (layer "F.Cu") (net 8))
 (segment (start 158.585284 115.449988) (end 158.251008 115.449988) (width 0.25) (layer "F.Cu") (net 8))
 (segment (start 168.505 116.425) (end 168.505 117.4) (width 0.25) (layer "F.Cu") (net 8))
 (segment (start 159.735296 116.6) (end 158.585284 115.449988) (width 0.25) (layer "F.Cu") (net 8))
 (segment (start 157.300996 116.4) (end 156.753553 116.4) (width 0.25) (layer "F.Cu") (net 8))
 (segment (start 162.4343 116.6) (end 159.735296 116.6) (width 0.25) (layer "F.Cu") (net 8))
 (segment (start 165.3 118.9) (end 162.599989 116.199989) (width 0.25) (layer "F.Cu") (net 7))
 (segment (start 158.700996 115) (end 157.656497 115) (width 0.25) (layer "F.Cu") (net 7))
 (segment (start 167.235 117.245689) (end 165.580689 118.9) (width 0.25) (layer "F.Cu") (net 7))
 (segment (start 157.656497 115) (end 156.858579 115.797918) (width 0.25) (layer "F.Cu") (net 7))
 (segment (start 159.900985 116.199989) (end 158.700996 115) (width 0.25) (layer "F.Cu") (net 7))
 (segment (start 165.580689 118.9) (end 165.3 118.9) (width 0.25) (layer "F.Cu") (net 7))
 (segment (start 162.599989 116.199989) (end 159.900985 116.199989) (width 0.25) (layer "F.Cu") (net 7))
 (segment (start 167.235 116.425) (end 167.235 117.245689) (width 0.25) (layer "F.Cu") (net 7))
 (segment (start 173.8875 124.4) (end 172.6875 123.2) (width 0.25) (layer "F.Cu") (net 9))
 (segment (start 167.235 121.375) (end 167.235 119.765) (width 0.25) (layer "F.Cu") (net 9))
 (segment (start 167.235 119.765) (end 168.5 118.5) (width 0.25) (layer "F.Cu") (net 9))
 (segment (start 172.6875 123.2) (end 172.1 123.2) (width 0.25) (layer "F.Cu") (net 9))
 (via (at 168.5 118.5) (size 0.8) (drill 0.4) (layers "F.Cu" "B.Cu") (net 9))
 (via (at 172.1 123.2) (size 0.8) (drill 0.4) (layers "F.Cu" "B.Cu") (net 9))
 (segment (start 168.5 118.5) (end 172.1 122.1) (width 0.25) (layer "B.Cu") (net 9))
 (segment (start 172.1 122.1) (end 172.1 123.2) (width 0.25) (layer "B.Cu") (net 9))
 (segment (start 172.3125 124.4) (end 170.7875 124.4) (width 0.25) (layer "F.Cu") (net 3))
 (segment (start 157.494975 117.848528) (end 157.681596 118.035149) (width 0.25) (layer "F.Cu") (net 5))
 (segment (start 157.681596 118.718404) (end 156.4 120) (width 0.25) (layer "F.Cu") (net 5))
 (segment (start 157.681596 118.035149) (end 157.681596 118.718404) (width 0.25) (layer "F.Cu") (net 5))
 (segment (start 158.618404 117.681596) (end 159.124976 117.175024) (width 0.25) (layer "F.Cu") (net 6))
 (segment (start 163.1 119.1) (end 163.1 120) (width 0.25) (layer "F.Cu") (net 6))
 (segment (start 158.035149 117.681596) (end 158.618404 117.681596) (width 0.25) (layer "F.Cu") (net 6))
 (segment (start 161.175024 117.175024) (end 163.1 119.1) (width 0.25) (layer "F.Cu") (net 6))
 (segment (start 159.124976 117.175024) (end 161.175024 117.175024) (width 0.25) (layer "F.Cu") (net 6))
 (segment (start 157.848528 117.494975) (end 158.035149 117.681596) (width 0.25) (layer "F.Cu") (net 6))
 (segment (start 165.965 120.080391) (end 166.896916 119.148475) (width 0.25) (layer "F.Cu") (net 13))
 (segment (start 165.965 121.375) (end 165.965 120.080391) (width 0.25) (layer "F.Cu") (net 13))
 (via (at 166.896916 119.148475) (size 0.8) (drill 0.4) (layers "F.Cu" "B.Cu") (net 13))
 (segment (start 166.896916 120.646916) (end 166.896916 119.148475) (width 0.25) (layer "B.Cu") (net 13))
 (segment (start 167.9 121.65) (end 166.896916 120.646916) (width 0.25) (layer "B.Cu") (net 13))
 (segment (start 165.965 115.45) (end 166.24001 115.17499) (width 0.25) (layer "F.Cu") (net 11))
 (segment (start 166.24001 115.17499) (end 170.04999 115.17499) (width 0.25) (layer "F.Cu") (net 11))
 (segment (start 170.04999 115.17499) (end 170.575 115.7) (width 0.25) (layer "F.Cu") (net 11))
 (segment (start 165.965 116.425) (end 165.965 115.45) (width 0.25) (layer "F.Cu") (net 11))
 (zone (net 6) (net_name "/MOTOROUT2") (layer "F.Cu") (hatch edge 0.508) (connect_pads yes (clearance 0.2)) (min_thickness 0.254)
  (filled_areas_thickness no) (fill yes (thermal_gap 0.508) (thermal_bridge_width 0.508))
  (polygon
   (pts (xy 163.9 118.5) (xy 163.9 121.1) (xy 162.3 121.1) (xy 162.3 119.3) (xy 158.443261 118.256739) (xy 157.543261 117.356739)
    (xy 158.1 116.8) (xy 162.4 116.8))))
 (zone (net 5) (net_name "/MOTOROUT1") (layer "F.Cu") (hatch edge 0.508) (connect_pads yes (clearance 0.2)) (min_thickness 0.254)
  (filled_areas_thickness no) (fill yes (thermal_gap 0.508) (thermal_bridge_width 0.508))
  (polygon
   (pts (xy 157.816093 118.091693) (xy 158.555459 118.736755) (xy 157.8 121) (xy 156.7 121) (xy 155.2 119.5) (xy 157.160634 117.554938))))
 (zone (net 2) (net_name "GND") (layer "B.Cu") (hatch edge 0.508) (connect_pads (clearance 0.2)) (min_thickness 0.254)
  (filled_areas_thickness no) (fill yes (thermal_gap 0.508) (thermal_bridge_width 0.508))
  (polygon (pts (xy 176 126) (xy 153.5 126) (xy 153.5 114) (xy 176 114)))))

